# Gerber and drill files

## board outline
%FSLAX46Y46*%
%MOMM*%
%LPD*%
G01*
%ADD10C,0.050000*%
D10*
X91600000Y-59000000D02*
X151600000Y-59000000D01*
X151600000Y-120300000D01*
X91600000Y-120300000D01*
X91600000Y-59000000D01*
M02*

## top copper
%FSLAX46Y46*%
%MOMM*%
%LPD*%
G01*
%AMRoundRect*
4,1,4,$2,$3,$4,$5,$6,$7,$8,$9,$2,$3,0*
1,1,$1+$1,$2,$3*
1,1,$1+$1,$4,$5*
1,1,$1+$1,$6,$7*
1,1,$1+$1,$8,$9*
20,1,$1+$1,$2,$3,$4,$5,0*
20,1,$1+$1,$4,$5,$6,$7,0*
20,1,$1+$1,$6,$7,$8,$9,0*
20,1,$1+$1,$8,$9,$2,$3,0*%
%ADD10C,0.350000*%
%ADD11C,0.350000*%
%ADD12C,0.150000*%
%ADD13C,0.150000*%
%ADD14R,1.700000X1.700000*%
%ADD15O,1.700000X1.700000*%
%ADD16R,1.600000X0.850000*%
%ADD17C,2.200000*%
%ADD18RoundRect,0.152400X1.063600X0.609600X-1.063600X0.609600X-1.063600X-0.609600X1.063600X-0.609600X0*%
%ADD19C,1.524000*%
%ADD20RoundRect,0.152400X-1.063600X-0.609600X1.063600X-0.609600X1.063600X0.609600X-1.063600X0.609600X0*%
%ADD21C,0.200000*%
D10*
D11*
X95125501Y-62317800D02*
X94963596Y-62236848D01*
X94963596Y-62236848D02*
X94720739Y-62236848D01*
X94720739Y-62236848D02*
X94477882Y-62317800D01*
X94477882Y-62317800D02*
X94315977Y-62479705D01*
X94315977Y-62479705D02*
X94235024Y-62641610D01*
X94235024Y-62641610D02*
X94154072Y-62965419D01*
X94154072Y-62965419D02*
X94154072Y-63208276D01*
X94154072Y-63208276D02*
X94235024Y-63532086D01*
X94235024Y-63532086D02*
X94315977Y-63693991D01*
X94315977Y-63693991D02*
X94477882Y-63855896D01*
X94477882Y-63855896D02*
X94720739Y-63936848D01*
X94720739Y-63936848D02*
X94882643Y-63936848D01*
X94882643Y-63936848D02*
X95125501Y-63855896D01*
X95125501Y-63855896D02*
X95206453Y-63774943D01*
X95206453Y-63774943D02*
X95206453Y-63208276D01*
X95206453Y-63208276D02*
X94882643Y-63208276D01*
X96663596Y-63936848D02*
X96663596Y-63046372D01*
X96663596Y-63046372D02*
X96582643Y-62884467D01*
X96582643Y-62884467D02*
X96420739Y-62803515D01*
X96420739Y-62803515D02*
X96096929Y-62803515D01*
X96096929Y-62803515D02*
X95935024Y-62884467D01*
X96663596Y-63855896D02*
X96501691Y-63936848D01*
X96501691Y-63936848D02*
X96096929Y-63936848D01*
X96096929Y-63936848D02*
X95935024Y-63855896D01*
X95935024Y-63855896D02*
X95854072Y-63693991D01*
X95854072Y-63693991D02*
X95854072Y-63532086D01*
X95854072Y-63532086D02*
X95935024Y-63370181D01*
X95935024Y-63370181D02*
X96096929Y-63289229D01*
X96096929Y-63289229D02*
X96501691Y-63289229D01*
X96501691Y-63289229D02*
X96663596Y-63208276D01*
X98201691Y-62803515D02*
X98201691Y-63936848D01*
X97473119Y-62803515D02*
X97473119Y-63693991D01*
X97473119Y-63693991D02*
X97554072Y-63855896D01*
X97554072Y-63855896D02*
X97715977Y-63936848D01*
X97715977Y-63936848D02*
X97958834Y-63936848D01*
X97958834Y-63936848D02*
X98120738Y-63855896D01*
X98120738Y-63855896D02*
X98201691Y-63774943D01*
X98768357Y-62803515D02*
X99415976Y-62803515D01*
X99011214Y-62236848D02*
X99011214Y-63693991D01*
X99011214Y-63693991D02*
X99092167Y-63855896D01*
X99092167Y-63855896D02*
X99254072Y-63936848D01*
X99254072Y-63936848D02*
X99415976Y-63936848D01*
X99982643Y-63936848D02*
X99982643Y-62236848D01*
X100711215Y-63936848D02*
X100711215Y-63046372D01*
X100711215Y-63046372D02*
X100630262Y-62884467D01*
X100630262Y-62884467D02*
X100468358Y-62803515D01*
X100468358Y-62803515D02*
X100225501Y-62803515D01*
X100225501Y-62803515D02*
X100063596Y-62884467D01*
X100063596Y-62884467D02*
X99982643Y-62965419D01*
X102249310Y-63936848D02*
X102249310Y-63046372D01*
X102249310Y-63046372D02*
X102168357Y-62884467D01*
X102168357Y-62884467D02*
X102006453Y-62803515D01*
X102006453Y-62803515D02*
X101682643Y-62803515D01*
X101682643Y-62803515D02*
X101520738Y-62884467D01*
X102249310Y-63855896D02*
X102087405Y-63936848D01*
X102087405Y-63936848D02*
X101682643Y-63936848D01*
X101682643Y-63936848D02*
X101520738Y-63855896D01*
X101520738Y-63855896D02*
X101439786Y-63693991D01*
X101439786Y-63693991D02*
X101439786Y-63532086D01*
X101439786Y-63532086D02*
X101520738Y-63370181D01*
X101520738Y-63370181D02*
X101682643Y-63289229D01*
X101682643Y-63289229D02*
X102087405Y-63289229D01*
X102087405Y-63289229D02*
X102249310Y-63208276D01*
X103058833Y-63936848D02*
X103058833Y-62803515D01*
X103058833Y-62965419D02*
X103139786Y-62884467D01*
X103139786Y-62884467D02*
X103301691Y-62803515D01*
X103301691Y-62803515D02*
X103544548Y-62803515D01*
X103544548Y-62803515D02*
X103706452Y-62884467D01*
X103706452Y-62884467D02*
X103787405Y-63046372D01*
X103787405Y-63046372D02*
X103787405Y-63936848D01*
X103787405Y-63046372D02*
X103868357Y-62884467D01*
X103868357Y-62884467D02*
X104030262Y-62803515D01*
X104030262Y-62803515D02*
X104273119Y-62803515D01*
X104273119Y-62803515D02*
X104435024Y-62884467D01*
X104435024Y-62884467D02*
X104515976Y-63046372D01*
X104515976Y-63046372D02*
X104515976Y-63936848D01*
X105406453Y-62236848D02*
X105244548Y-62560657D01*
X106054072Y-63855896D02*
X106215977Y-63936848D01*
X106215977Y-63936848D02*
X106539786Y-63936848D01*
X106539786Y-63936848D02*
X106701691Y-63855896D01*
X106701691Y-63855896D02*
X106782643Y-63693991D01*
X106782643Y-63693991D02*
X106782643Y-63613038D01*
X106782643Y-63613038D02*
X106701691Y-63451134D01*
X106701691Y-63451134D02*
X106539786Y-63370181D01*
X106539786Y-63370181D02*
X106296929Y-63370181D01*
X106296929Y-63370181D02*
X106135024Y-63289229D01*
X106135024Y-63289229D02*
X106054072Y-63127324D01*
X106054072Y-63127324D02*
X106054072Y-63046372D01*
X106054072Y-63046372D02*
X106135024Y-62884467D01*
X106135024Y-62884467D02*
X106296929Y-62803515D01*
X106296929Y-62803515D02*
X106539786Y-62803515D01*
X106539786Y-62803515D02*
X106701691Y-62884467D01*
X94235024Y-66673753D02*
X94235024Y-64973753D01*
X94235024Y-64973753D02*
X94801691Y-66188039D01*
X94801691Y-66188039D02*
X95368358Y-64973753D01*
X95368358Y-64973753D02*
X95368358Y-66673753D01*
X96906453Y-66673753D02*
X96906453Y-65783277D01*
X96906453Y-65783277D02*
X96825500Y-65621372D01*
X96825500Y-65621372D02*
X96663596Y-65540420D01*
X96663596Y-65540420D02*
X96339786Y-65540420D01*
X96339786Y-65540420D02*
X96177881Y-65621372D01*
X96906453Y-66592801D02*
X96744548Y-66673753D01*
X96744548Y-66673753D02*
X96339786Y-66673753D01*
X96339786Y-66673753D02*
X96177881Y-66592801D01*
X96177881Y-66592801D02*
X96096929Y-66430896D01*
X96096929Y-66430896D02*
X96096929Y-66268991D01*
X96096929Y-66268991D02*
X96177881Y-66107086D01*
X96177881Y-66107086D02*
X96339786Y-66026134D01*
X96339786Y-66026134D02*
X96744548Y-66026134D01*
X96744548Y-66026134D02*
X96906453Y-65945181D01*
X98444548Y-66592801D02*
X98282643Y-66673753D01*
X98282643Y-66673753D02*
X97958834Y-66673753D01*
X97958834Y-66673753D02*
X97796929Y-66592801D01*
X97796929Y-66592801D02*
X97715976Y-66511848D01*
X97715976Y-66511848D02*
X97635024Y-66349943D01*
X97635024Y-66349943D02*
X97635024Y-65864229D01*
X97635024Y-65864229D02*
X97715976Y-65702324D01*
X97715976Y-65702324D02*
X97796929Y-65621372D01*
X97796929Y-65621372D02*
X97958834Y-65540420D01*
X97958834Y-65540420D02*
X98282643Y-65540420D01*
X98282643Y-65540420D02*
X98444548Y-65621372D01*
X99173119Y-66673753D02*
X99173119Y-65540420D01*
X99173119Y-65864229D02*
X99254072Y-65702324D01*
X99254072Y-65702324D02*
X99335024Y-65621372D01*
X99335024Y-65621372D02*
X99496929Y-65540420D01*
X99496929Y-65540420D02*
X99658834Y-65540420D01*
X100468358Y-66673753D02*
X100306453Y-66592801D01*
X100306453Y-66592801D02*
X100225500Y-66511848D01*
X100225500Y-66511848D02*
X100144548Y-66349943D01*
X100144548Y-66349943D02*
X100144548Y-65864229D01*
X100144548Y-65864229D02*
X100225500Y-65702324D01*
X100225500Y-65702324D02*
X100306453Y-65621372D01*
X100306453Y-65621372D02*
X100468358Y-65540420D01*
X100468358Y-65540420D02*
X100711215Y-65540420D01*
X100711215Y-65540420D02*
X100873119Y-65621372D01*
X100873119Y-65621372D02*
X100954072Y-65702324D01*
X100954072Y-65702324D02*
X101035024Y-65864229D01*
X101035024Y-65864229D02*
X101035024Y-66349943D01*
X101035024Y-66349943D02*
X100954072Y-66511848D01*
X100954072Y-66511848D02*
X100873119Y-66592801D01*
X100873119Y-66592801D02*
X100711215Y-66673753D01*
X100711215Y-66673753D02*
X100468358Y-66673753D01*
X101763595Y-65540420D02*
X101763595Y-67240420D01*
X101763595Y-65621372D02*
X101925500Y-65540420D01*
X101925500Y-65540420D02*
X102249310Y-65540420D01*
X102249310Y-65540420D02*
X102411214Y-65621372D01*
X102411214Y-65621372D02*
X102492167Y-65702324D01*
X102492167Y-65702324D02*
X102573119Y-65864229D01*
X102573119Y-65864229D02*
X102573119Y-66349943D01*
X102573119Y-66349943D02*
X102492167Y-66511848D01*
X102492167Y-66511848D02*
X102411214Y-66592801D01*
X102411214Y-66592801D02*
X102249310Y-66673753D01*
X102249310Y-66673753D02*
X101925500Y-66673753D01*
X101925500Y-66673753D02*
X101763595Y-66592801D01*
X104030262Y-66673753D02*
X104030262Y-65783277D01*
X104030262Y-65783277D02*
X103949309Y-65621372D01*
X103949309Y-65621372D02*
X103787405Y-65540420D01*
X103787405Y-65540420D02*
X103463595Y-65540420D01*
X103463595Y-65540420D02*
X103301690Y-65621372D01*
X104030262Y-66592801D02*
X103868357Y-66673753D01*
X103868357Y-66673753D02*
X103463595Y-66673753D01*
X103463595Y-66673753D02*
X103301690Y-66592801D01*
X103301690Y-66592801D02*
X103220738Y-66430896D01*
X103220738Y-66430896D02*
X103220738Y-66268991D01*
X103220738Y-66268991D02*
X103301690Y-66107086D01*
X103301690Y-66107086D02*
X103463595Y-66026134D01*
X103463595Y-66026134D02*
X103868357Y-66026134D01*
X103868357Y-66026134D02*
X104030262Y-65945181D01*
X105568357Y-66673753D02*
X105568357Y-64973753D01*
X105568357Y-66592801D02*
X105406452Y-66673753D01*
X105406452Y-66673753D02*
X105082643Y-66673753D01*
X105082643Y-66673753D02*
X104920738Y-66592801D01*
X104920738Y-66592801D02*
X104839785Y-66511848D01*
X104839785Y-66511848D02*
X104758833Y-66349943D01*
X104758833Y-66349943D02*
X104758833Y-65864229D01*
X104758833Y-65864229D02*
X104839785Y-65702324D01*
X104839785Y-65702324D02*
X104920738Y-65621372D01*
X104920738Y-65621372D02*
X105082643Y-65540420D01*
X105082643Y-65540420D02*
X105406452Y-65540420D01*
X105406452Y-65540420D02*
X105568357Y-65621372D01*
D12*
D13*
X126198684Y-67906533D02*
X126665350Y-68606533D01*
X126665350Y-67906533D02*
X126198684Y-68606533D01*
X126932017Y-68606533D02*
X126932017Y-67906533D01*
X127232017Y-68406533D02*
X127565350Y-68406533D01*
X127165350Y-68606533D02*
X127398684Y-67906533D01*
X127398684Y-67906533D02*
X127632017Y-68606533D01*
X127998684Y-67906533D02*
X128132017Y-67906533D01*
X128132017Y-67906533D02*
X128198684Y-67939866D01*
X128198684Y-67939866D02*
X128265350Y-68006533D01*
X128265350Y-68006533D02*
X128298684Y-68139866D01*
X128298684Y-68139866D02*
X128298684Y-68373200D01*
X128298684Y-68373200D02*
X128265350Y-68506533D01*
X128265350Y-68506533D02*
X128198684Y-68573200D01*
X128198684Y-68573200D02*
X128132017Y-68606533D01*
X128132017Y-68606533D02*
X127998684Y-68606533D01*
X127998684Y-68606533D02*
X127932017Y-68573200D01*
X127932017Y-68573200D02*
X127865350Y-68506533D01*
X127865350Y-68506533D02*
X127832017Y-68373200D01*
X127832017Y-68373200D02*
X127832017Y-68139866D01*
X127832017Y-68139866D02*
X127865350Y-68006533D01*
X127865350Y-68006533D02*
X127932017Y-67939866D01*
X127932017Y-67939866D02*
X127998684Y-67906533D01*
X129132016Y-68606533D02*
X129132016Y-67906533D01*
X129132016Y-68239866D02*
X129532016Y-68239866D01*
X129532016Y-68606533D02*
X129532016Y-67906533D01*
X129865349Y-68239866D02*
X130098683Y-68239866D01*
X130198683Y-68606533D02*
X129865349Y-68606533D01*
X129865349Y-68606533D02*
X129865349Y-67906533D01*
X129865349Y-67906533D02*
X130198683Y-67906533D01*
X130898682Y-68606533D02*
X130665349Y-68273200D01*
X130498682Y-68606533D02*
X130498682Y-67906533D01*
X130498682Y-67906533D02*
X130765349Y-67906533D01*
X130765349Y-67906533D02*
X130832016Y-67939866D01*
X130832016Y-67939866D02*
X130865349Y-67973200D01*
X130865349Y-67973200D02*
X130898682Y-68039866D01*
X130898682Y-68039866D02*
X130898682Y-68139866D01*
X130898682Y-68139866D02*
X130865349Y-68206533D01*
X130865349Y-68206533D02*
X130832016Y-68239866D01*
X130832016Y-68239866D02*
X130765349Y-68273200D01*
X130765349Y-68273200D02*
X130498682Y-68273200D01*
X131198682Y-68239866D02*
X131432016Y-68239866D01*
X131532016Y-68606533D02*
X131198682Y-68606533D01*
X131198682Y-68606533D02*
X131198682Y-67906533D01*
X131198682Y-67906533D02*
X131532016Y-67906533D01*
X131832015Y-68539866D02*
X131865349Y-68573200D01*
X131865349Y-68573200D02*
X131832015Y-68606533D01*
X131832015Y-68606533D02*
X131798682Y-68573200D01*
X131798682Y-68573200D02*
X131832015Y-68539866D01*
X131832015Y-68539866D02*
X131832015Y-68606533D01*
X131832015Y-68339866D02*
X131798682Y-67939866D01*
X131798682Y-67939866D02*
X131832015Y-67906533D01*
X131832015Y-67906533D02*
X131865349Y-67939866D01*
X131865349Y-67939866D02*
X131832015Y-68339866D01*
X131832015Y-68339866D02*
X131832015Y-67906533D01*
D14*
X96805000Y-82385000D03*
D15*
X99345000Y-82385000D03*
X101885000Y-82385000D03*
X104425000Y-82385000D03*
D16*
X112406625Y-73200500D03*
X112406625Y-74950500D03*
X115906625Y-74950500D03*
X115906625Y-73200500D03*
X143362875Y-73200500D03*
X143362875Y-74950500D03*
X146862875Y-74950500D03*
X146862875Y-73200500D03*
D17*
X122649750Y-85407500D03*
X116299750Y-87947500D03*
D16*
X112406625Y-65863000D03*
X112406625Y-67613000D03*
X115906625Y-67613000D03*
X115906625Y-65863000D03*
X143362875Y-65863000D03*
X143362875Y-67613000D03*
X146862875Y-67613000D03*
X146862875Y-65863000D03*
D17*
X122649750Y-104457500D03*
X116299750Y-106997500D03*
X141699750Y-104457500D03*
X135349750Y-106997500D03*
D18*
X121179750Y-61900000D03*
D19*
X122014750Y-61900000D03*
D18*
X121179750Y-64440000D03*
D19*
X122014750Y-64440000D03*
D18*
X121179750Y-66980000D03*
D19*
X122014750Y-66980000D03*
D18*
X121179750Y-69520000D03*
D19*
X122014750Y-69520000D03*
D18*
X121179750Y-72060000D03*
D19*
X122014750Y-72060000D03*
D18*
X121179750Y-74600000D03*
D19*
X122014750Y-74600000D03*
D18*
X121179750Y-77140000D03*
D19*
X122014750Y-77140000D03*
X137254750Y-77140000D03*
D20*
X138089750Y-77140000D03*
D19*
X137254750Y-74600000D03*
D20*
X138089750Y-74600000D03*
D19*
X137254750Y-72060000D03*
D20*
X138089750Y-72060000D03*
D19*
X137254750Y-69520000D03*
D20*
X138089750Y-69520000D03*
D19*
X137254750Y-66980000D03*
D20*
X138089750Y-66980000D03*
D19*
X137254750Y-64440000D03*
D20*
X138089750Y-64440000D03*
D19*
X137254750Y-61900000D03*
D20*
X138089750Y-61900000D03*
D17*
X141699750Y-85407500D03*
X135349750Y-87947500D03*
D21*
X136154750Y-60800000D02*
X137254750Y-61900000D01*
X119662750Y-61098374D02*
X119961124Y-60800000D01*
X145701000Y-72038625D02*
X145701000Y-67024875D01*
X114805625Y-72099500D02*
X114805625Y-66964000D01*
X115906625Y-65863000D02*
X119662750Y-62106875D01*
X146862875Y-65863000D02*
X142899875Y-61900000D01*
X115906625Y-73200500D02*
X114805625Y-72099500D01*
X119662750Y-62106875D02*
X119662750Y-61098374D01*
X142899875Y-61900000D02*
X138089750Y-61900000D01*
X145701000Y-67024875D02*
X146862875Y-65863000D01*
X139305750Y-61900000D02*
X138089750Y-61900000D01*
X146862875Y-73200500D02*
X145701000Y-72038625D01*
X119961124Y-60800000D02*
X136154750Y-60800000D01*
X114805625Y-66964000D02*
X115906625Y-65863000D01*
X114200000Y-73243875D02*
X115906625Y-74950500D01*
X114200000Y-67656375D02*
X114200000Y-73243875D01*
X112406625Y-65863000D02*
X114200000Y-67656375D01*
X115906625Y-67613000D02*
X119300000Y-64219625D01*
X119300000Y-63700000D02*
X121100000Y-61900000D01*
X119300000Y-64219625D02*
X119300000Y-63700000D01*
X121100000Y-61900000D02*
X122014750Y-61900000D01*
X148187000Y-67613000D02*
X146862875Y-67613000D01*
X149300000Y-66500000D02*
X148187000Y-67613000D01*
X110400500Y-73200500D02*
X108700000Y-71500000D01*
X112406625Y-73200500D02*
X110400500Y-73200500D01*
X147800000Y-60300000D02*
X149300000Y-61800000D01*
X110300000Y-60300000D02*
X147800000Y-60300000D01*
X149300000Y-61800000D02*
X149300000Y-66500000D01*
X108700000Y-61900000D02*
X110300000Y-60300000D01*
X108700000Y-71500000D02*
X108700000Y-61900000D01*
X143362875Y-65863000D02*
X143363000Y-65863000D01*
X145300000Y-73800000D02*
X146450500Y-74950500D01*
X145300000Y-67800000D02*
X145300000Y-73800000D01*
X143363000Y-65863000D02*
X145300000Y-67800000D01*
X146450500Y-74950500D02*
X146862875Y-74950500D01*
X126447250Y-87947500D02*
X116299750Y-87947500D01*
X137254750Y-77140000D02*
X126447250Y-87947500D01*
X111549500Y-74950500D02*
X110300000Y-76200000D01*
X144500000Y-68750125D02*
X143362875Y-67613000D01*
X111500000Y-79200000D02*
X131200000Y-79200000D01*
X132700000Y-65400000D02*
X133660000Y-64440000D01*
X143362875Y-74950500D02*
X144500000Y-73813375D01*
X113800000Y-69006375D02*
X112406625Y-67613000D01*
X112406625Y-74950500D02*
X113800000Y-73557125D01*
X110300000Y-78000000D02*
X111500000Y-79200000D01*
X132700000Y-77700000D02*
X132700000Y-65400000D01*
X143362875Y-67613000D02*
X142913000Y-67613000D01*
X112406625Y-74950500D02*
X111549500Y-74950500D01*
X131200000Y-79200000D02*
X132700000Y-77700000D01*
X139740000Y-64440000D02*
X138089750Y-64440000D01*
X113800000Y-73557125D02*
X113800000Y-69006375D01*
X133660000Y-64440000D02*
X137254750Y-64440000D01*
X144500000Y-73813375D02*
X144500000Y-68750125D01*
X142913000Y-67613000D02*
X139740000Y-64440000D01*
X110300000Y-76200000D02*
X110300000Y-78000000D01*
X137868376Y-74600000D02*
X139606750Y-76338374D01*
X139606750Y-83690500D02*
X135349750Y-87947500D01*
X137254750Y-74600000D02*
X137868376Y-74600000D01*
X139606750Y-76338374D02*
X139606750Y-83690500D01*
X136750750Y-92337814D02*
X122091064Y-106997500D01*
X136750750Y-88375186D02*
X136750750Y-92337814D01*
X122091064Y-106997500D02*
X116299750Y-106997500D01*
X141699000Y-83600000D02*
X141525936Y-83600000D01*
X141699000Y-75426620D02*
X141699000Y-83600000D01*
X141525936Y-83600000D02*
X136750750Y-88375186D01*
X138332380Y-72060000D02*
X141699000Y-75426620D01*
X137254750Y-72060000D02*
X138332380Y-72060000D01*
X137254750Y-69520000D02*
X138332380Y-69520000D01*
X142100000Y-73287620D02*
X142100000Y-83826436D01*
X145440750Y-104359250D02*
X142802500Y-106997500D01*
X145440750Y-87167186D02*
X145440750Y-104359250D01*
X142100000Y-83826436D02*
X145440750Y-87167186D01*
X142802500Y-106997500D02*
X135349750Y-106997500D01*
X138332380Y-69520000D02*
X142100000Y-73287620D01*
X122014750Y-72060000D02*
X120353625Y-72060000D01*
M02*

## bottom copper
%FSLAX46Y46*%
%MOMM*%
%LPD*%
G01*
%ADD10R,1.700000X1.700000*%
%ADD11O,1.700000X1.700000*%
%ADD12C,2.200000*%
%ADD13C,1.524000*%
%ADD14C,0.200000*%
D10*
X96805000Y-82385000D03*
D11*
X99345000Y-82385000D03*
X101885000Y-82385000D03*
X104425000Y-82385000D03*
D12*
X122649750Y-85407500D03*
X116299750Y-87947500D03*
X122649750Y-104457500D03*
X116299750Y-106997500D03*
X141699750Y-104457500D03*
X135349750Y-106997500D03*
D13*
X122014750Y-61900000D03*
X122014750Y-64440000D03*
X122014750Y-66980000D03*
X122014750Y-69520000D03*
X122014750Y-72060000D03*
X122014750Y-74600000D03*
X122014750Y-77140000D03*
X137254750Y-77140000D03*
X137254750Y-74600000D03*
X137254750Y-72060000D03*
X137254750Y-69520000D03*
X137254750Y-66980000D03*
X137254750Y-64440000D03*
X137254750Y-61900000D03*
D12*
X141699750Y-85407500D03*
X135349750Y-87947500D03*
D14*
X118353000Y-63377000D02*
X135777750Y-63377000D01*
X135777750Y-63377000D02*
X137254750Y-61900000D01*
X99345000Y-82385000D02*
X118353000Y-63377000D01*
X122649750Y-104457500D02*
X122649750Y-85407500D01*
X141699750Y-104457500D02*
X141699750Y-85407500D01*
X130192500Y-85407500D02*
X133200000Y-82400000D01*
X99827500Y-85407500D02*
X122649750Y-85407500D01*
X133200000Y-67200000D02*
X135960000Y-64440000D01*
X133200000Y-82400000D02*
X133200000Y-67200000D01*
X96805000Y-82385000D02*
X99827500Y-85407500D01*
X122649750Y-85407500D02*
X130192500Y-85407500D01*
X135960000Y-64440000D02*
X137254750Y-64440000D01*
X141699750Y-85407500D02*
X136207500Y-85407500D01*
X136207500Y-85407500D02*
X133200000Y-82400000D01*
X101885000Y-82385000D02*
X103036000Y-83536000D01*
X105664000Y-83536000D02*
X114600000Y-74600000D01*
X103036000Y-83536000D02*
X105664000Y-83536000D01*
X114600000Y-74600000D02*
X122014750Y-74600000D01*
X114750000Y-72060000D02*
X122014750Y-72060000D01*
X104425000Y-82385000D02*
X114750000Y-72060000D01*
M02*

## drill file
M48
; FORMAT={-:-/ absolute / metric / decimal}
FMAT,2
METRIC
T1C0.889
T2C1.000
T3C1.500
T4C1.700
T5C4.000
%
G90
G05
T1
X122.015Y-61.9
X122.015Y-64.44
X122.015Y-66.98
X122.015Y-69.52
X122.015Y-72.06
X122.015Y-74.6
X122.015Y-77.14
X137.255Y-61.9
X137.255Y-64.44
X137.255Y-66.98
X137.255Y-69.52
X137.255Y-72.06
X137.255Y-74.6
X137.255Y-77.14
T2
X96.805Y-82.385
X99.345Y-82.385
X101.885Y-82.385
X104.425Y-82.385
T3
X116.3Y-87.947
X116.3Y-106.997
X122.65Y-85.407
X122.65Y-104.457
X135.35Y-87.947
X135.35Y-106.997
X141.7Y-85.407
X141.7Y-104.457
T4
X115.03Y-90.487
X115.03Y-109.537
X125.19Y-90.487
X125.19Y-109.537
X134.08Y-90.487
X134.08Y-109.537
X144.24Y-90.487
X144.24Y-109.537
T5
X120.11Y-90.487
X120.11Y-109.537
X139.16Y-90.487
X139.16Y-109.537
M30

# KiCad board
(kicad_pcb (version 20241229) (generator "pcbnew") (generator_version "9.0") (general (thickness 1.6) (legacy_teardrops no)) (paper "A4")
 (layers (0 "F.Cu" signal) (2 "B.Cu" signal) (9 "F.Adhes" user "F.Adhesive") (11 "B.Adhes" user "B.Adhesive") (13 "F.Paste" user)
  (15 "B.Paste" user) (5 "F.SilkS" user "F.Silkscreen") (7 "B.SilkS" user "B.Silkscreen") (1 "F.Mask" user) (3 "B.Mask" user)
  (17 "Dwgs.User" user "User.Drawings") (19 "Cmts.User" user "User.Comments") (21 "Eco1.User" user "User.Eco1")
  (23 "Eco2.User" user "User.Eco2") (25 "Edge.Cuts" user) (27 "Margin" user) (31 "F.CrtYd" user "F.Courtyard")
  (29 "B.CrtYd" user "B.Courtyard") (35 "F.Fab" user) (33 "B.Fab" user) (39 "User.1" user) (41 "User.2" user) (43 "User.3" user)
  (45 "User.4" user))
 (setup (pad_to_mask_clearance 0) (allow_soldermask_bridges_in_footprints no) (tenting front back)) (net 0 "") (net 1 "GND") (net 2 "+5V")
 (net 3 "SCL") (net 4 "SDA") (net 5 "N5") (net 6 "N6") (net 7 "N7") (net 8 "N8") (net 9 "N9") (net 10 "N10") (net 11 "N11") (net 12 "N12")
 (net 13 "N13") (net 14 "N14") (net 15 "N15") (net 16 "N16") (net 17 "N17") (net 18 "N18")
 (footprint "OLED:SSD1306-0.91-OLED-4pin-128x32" (layer "F.Cu") (at 94.615 118.885 90)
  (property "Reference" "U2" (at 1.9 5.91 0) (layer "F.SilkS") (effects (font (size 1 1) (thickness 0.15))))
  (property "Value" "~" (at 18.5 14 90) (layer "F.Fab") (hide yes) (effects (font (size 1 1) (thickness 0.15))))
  (pad "1" thru_hole rect (at 36.5 2.19 90) (size 1.7 1.7) (drill 1) (layers "*.Cu" "*.Mask") (remove_unused_layers no) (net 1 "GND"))
  (pad "2" thru_hole oval (at 36.5 4.73 90) (size 1.7 1.7) (drill 1) (layers "*.Cu" "*.Mask") (remove_unused_layers no) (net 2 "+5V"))
  (pad "3" thru_hole oval (at 36.5 7.27 90) (size 1.7 1.7) (drill 1) (layers "*.Cu" "*.Mask") (remove_unused_layers no) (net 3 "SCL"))
  (pad "4" thru_hole oval (at 36.5 9.81 90) (size 1.7 1.7) (drill 1) (layers "*.Cu" "*.Mask") (remove_unused_layers no) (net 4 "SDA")))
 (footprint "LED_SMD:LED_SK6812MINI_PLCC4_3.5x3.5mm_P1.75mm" (layer "F.Cu") (at 114.156625 74.0755)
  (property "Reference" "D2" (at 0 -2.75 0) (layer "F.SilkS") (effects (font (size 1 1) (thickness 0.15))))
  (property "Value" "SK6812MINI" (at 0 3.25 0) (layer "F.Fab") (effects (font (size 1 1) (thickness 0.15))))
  (pad "1" smd rect (at -1.75 -0.875) (size 1.6 0.85) (layers "F.Cu" "F.Mask" "F.Paste") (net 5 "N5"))
  (pad "2" smd rect (at -1.75 0.875) (size 1.6 0.85) (layers "F.Cu" "F.Mask" "F.Paste") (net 1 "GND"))
  (pad "3" smd rect (at 1.75 0.875) (size 1.6 0.85) (layers "F.Cu" "F.Mask" "F.Paste") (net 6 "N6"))
  (pad "4" smd rect (at 1.75 -0.875) (size 1.6 0.85) (layers "F.Cu" "F.Mask" "F.Paste") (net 2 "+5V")))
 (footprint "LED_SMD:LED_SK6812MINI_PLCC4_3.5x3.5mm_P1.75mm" (layer "F.Cu") (at 145.112875 74.0755)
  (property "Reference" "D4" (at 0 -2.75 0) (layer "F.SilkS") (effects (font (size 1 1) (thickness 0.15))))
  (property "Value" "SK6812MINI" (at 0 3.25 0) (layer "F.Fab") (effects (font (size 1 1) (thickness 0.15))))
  (pad "1" smd rect (at -1.75 -0.875) (size 1.6 0.85) (layers "F.Cu" "F.Mask" "F.Paste") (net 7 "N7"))
  (pad "2" smd rect (at -1.75 0.875) (size 1.6 0.85) (layers "F.Cu" "F.Mask" "F.Paste") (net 1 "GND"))
  (pad "3" smd rect (at 1.75 0.875) (size 1.6 0.85) (layers "F.Cu" "F.Mask" "F.Paste") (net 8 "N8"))
  (pad "4" smd rect (at 1.75 -0.875) (size 1.6 0.85) (layers "F.Cu" "F.Mask" "F.Paste") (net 2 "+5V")))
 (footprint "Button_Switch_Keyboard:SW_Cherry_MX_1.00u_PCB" (layer "F.Cu") (at 122.64975 85.4075)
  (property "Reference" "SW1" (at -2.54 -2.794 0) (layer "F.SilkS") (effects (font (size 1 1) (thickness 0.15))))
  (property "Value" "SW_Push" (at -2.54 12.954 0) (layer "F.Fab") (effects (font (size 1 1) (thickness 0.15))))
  (pad "" np_thru_hole circle (at -7.62 5.08) (size 1.7 1.7) (drill 1.7) (layers "*.Cu" "*.Mask"))
  (pad "" np_thru_hole circle (at -2.54 5.08) (size 4 4) (drill 4) (layers "*.Cu" "*.Mask"))
  (pad "" np_thru_hole circle (at 2.54 5.08) (size 1.7 1.7) (drill 1.7) (layers "*.Cu" "*.Mask"))
  (pad "1" thru_hole circle (at 0 0) (size 2.2 2.2) (drill 1.5) (layers "*.Cu" "*.Mask") (remove_unused_layers no) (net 1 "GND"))
  (pad "2" thru_hole circle (at -6.35 2.54) (size 2.2 2.2) (drill 1.5) (layers "*.Cu" "*.Mask") (remove_unused_layers no) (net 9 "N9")))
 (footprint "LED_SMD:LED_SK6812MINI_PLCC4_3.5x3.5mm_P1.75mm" (layer "F.Cu") (at 114.156625 66.738)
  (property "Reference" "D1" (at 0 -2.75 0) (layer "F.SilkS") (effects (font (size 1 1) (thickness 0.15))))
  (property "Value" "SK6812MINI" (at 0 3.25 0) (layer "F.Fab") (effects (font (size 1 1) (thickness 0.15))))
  (pad "1" smd rect (at -1.75 -0.875) (size 1.6 0.85) (layers "F.Cu" "F.Mask" "F.Paste") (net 6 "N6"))
  (pad "2" smd rect (at -1.75 0.875) (size 1.6 0.85) (layers "F.Cu" "F.Mask" "F.Paste") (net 1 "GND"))
  (pad "3" smd rect (at 1.75 0.875) (size 1.6 0.85) (layers "F.Cu" "F.Mask" "F.Paste") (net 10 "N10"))
  (pad "4" smd rect (at 1.75 -0.875) (size 1.6 0.85) (layers "F.Cu" "F.Mask" "F.Paste") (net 2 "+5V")))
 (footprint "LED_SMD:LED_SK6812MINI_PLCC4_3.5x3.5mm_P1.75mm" (layer "F.Cu") (at 145.112875 66.738)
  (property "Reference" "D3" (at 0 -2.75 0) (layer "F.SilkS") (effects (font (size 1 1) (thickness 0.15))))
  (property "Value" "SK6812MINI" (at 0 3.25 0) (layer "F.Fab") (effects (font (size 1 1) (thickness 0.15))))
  (pad "1" smd rect (at -1.75 -0.875) (size 1.6 0.85) (layers "F.Cu" "F.Mask" "F.Paste") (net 8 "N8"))
  (pad "2" smd rect (at -1.75 0.875) (size 1.6 0.85) (layers "F.Cu" "F.Mask" "F.Paste") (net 1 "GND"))
  (pad "3" smd rect (at 1.75 0.875) (size 1.6 0.85) (layers "F.Cu" "F.Mask" "F.Paste") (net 5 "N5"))
  (pad "4" smd rect (at 1.75 -0.875) (size 1.6 0.85) (layers "F.Cu" "F.Mask" "F.Paste") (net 2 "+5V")))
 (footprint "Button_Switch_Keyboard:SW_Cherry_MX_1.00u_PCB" (layer "F.Cu") (at 122.64975 104.4575)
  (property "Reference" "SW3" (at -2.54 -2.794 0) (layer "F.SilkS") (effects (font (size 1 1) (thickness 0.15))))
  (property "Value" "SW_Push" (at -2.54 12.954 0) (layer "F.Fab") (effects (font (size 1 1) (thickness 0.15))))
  (pad "" np_thru_hole circle (at -7.62 5.08) (size 1.7 1.7) (drill 1.7) (layers "*.Cu" "*.Mask"))
  (pad "" np_thru_hole circle (at -2.54 5.08) (size 4 4) (drill 4) (layers "*.Cu" "*.Mask"))
  (pad "" np_thru_hole circle (at 2.54 5.08) (size 1.7 1.7) (drill 1.7) (layers "*.Cu" "*.Mask"))
  (pad "1" thru_hole circle (at 0 0) (size 2.2 2.2) (drill 1.5) (layers "*.Cu" "*.Mask") (remove_unused_layers no) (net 1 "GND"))
  (pad "2" thru_hole circle (at -6.35 2.54) (size 2.2 2.2) (drill 1.5) (layers "*.Cu" "*.Mask") (remove_unused_layers no) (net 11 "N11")))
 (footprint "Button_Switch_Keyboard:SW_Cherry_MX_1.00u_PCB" (layer "F.Cu") (at 141.69975 104.4575)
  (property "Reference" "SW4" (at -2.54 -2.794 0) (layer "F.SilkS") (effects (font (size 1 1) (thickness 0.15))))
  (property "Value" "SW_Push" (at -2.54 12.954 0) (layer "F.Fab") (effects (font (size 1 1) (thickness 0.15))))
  (pad "" np_thru_hole circle (at -7.62 5.08) (size 1.7 1.7) (drill 1.7) (layers "*.Cu" "*.Mask"))
  (pad "" np_thru_hole circle (at -2.54 5.08) (size 4 4) (drill 4) (layers "*.Cu" "*.Mask"))
  (pad "" np_thru_hole circle (at 2.54 5.08) (size 1.7 1.7) (drill 1.7) (layers "*.Cu" "*.Mask"))
  (pad "1" thru_hole circle (at 0 0) (size 2.2 2.2) (drill 1.5) (layers "*.Cu" "*.Mask") (remove_unused_layers no) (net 1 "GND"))
  (pad "2" thru_hole circle (at -6.35 2.54) (size 2.2 2.2) (drill 1.5) (layers "*.Cu" "*.Mask") (remove_unused_layers no) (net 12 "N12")))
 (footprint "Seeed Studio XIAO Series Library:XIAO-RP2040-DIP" (layer "F.Cu") (at 129.63475 69.52)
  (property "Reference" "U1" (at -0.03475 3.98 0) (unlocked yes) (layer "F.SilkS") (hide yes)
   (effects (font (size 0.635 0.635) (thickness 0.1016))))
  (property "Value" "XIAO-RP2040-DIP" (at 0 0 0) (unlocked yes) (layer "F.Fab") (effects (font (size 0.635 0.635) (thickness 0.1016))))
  (pad "1" smd roundrect (at -8.455 -7.62 180) (size 2.432 1.524) (layers "F.Cu" "F.Mask") (roundrect_rratio 0.1) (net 10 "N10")
   (thermal_bridge_angle 45))
  (pad "1" thru_hole circle (at -7.62 -7.62 180) (size 1.524 1.524) (drill 0.889) (layers "*.Cu" "*.Mask") (remove_unused_layers no)
   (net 10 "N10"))
  (pad "2" smd roundrect (at -8.455 -5.08 180) (size 2.432 1.524) (layers "F.Cu" "F.Mask") (roundrect_rratio 0.1) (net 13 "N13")
   (thermal_bridge_angle 45))
  (pad "2" thru_hole circle (at -7.62 -5.08 180) (size 1.524 1.524) (drill 0.889) (layers "*.Cu" "*.Mask") (remove_unused_layers no)
   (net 13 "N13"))
  (pad "3" smd roundrect (at -8.455 -2.54 180) (size 2.432 1.524) (layers "F.Cu" "F.Mask") (roundrect_rratio 0.1) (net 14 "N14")
   (thermal_bridge_angle 45))
  (pad "3" thru_hole circle (at -7.62 -2.54 180) (size 1.524 1.524) (drill 0.889) (layers "*.Cu" "*.Mask") (remove_unused_layers no)
   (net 14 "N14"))
  (pad "4" smd roundrect (at -8.455 0 180) (size 2.432 1.524) (layers "F.Cu" "F.Mask") (roundrect_rratio 0.1) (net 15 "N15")
   (thermal_bridge_angle 45))
  (pad "4" thru_hole circle (at -7.62 0 180) (size 1.524 1.524) (drill 0.889) (layers "*.Cu" "*.Mask") (remove_unused_layers no)
   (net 15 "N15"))
  (pad "5" smd roundrect (at -8.455 2.54 180) (size 2.432 1.524) (layers "F.Cu" "F.Mask") (roundrect_rratio 0.1) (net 4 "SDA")
   (thermal_bridge_angle 45))
  (pad "5" thru_hole circle (at -7.62 2.54 180) (size 1.524 1.524) (drill 0.889) (layers "*.Cu" "*.Mask") (remove_unused_layers no)
   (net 4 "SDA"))
  (pad "6" smd roundrect (at -8.455 5.08 180) (size 2.432 1.524) (layers "F.Cu" "F.Mask") (roundrect_rratio 0.1) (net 3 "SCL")
   (thermal_bridge_angle 45))
  (pad "6" thru_hole circle (at -7.62 5.08 180) (size 1.524 1.524) (drill 0.889) (layers "*.Cu" "*.Mask") (remove_unused_layers no)
   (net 3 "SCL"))
  (pad "7" smd roundrect (at -8.455 7.62 180) (size 2.432 1.524) (layers "F.Cu" "F.Mask") (roundrect_rratio 0.1) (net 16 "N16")
   (thermal_bridge_angle 45))
  (pad "7" thru_hole circle (at -7.62 7.62 180) (size 1.524 1.524) (drill 0.889) (layers "*.Cu" "*.Mask") (remove_unused_layers no)
   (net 16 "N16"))
  (pad "8" thru_hole circle (at 7.62 7.62) (size 1.524 1.524) (drill 0.889) (layers "*.Cu" "*.Mask") (remove_unused_layers no) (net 9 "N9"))
  (pad "8" smd roundrect (at 8.455 7.62) (size 2.432 1.524) (layers "F.Cu" "F.Mask") (roundrect_rratio 0.1) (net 9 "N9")
   (thermal_bridge_angle 45))
  (pad "9" thru_hole circle (at 7.62 5.08) (size 1.524 1.524) (drill 0.889) (layers "*.Cu" "*.Mask") (remove_unused_layers no)
   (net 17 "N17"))
  (pad "9" smd roundrect (at 8.455 5.08) (size 2.432 1.524) (layers "F.Cu" "F.Mask") (roundrect_rratio 0.1) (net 17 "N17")
   (thermal_bridge_angle 45))
  (pad "10" thru_hole circle (at 7.62 2.54) (size 1.524 1.524) (drill 0.889) (layers "*.Cu" "*.Mask") (remove_unused_layers no)
   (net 11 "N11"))
  (pad "10" smd roundrect (at 8.455 2.54) (size 2.432 1.524) (layers "F.Cu" "F.Mask") (roundrect_rratio 0.1) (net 11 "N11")
   (thermal_bridge_angle 45))
  (pad "11" thru_hole circle (at 7.62 0) (size 1.524 1.524) (drill 0.889) (layers "*.Cu" "*.Mask") (remove_unused_layers no) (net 12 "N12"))
  (pad "11" smd roundrect (at 8.455 0) (size 2.432 1.524) (layers "F.Cu" "F.Mask") (roundrect_rratio 0.1) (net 12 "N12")
   (thermal_bridge_angle 45))
  (pad "12" thru_hole circle (at 7.62 -2.54) (size 1.524 1.524) (drill 0.889) (layers "*.Cu" "*.Mask") (remove_unused_layers no)
   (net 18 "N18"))
  (pad "12" smd roundrect (at 8.455 -2.54) (size 2.432 1.524) (layers "F.Cu" "F.Mask") (roundrect_rratio 0.1) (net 18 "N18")
   (thermal_bridge_angle 45))
  (pad "13" thru_hole circle (at 7.62 -5.08) (size 1.524 1.524) (drill 0.889) (layers "*.Cu" "*.Mask") (remove_unused_layers no)
   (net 1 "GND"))
  (pad "13" smd roundrect (at 8.455 -5.08) (size 2.432 1.524) (layers "F.Cu" "F.Mask") (roundrect_rratio 0.1) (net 1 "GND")
   (thermal_bridge_angle 45))
  (pad "14" thru_hole circle (at 7.62 -7.62) (size 1.524 1.524) (drill 0.889) (layers "*.Cu" "*.Mask") (remove_unused_layers no)
   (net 2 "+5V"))
  (pad "14" smd roundrect (at 8.455 -7.62) (size 2.432 1.524) (layers "F.Cu" "F.Mask") (roundrect_rratio 0.1) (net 2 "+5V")
   (thermal_bridge_angle 45)))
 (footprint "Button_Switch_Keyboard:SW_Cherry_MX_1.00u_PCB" (layer "F.Cu") (at 141.69975 85.4075)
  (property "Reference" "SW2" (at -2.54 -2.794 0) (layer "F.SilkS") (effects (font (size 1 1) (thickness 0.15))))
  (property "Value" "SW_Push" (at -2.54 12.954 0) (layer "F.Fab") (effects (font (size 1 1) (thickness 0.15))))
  (pad "" np_thru_hole circle (at -7.62 5.08) (size 1.7 1.7) (drill 1.7) (layers "*.Cu" "*.Mask"))
  (pad "" np_thru_hole circle (at -2.54 5.08) (size 4 4) (drill 4) (layers "*.Cu" "*.Mask"))
  (pad "" np_thru_hole circle (at 2.54 5.08) (size 1.7 1.7) (drill 1.7) (layers "*.Cu" "*.Mask"))
  (pad "1" thru_hole circle (at 0 0) (size 2.2 2.2) (drill 1.5) (layers "*.Cu" "*.Mask") (remove_unused_layers no) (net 1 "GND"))
  (pad "2" thru_hole circle (at -6.35 2.54) (size 2.2 2.2) (drill 1.5) (layers "*.Cu" "*.Mask") (remove_unused_layers no) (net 17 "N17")))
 (gr_rect (start 91.6 59) (end 151.6 120.3) (stroke (width 0.05) (type default)) (fill no) (layer "Edge.Cuts"))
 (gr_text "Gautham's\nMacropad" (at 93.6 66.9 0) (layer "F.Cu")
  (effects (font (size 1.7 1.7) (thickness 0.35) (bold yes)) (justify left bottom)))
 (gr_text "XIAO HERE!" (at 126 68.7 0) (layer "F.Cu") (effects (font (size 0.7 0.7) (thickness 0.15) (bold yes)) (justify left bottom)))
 (segment (start 136.15475 60.8) (end 137.25475 61.9) (width 0.2) (layer "F.Cu") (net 2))
 (segment (start 119.66275 61.098374) (end 119.961124 60.8) (width 0.2) (layer "F.Cu") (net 2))
 (segment (start 145.701 72.038625) (end 145.701 67.024875) (width 0.2) (layer "F.Cu") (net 2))
 (segment (start 114.805625 72.0995) (end 114.805625 66.964) (width 0.2) (layer "F.Cu") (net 2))
 (segment (start 115.906625 65.863) (end 119.66275 62.106875) (width 0.2) (layer "F.Cu") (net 2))
 (segment (start 146.862875 65.863) (end 142.899875 61.9) (width 0.2) (layer "F.Cu") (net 2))
 (segment (start 115.906625 73.2005) (end 114.805625 72.0995) (width 0.2) (layer "F.Cu") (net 2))
 (segment (start 119.66275 62.106875) (end 119.66275 61.098374) (width 0.2) (layer "F.Cu") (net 2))
 (segment (start 142.899875 61.9) (end 138.08975 61.9) (width 0.2) (layer "F.Cu") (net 2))
 (segment (start 145.701 67.024875) (end 146.862875 65.863) (width 0.2) (layer "F.Cu") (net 2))
 (segment (start 139.30575 61.9) (end 138.08975 61.9) (width 0.2) (layer "F.Cu") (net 2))
 (segment (start 146.862875 73.2005) (end 145.701 72.038625) (width 0.2) (layer "F.Cu") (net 2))
 (segment (start 119.961124 60.8) (end 136.15475 60.8) (width 0.2) (layer "F.Cu") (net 2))
 (segment (start 114.805625 66.964) (end 115.906625 65.863) (width 0.2) (layer "F.Cu") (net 2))
 (segment (start 118.353 63.377) (end 135.77775 63.377) (width 0.2) (layer "B.Cu") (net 2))
 (segment (start 135.77775 63.377) (end 137.25475 61.9) (width 0.2) (layer "B.Cu") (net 2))
 (segment (start 99.345 82.385) (end 118.353 63.377) (width 0.2) (layer "B.Cu") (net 2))
 (segment (start 114.2 73.243875) (end 115.906625 74.9505) (width 0.2) (layer "F.Cu") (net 6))
 (segment (start 114.2 67.656375) (end 114.2 73.243875) (width 0.2) (layer "F.Cu") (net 6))
 (segment (start 112.406625 65.863) (end 114.2 67.656375) (width 0.2) (layer "F.Cu") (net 6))
 (segment (start 115.906625 67.613) (end 119.3 64.219625) (width 0.2) (layer "F.Cu") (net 10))
 (segment (start 119.3 63.7) (end 121.1 61.9) (width 0.2) (layer "F.Cu") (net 10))
 (segment (start 119.3 64.219625) (end 119.3 63.7) (width 0.2) (layer "F.Cu") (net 10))
 (segment (start 121.1 61.9) (end 122.01475 61.9) (width 0.2) (layer "F.Cu") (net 10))
 (segment (start 148.187 67.613) (end 146.862875 67.613) (width 0.2) (layer "F.Cu") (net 5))
 (segment (start 149.3 66.5) (end 148.187 67.613) (width 0.2) (layer "F.Cu") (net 5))
 (segment (start 110.4005 73.2005) (end 108.7 71.5) (width 0.2) (layer "F.Cu") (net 5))
 (segment (start 112.406625 73.2005) (end 110.4005 73.2005) (width 0.2) (layer "F.Cu") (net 5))
 (segment (start 147.8 60.3) (end 149.3 61.8) (width 0.2) (layer "F.Cu") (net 5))
 (segment (start 110.3 60.3) (end 147.8 60.3) (width 0.2) (layer "F.Cu") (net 5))
 (segment (start 149.3 61.8) (end 149.3 66.5) (width 0.2) (layer "F.Cu") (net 5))
 (segment (start 108.7 61.9) (end 110.3 60.3) (width 0.2) (layer "F.Cu") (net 5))
 (segment (start 108.7 71.5) (end 108.7 61.9) (width 0.2) (layer "F.Cu") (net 5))
 (segment (start 143.362875 65.863) (end 143.363 65.863) (width 0.2) (layer "F.Cu") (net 8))
 (segment (start 145.3 73.8) (end 146.4505 74.9505) (width 0.2) (layer "F.Cu") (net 8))
 (segment (start 145.3 67.8) (end 145.3 73.8) (width 0.2) (layer "F.Cu") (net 8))
 (segment (start 143.363 65.863) (end 145.3 67.8) (width 0.2) (layer "F.Cu") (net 8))
 (segment (start 146.4505 74.9505) (end 146.862875 74.9505) (width 0.2) (layer "F.Cu") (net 8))
 (segment (start 126.44725 87.9475) (end 116.29975 87.9475) (width 0.2) (layer "F.Cu") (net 9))
 (segment (start 137.25475 77.14) (end 126.44725 87.9475) (width 0.2) (layer "F.Cu") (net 9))
 (segment (start 111.5495 74.9505) (end 110.3 76.2) (width 0.2) (layer "F.Cu") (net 1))
 (segment (start 144.5 68.750125) (end 143.362875 67.613) (width 0.2) (layer "F.Cu") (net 1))
 (segment (start 111.5 79.2) (end 131.2 79.2) (width 0.2) (layer "F.Cu") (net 1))
 (segment (start 132.7 65.4) (end 133.66 64.44) (width 0.2) (layer "F.Cu") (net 1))
 (segment (start 143.362875 74.9505) (end 144.5 73.813375) (width 0.2) (layer "F.Cu") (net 1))
 (segment (start 113.8 69.006375) (end 112.406625 67.613) (width 0.2) (layer "F.Cu") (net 1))
 (segment (start 112.406625 74.9505) (end 113.8 73.557125) (width 0.2) (layer "F.Cu") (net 1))
 (segment (start 110.3 78) (end 111.5 79.2) (width 0.2) (layer "F.Cu") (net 1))
 (segment (start 132.7 77.7) (end 132.7 65.4) (width 0.2) (layer "F.Cu") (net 1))
 (segment (start 143.362875 67.613) (end 142.913 67.613) (width 0.2) (layer "F.Cu") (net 1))
 (segment (start 112.406625 74.9505) (end 111.5495 74.9505) (width 0.2) (layer "F.Cu") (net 1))
 (segment (start 131.2 79.2) (end 132.7 77.7) (width 0.2) (layer "F.Cu") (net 1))
 (segment (start 139.74 64.44) (end 138.08975 64.44) (width 0.2) (layer "F.Cu") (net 1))
 (segment (start 113.8 73.557125) (end 113.8 69.006375) (width 0.2) (layer "F.Cu") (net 1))
 (segment (start 133.66 64.44) (end 137.25475 64.44) (width 0.2) (layer "F.Cu") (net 1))
 (segment (start 144.5 73.813375) (end 144.5 68.750125) (width 0.2) (layer "F.Cu") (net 1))
 (segment (start 142.913 67.613) (end 139.74 64.44) (width 0.2) (layer "F.Cu") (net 1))
 (segment (start 110.3 76.2) (end 110.3 78) (width 0.2) (layer "F.Cu") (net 1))
 (segment (start 122.64975 104.4575) (end 122.64975 85.4075) (width 0.2) (layer "B.Cu") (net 1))
 (segment (start 141.69975 104.4575) (end 141.69975 85.4075) (width 0.2) (layer "B.Cu") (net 1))
 (segment (start 130.1925 85.4075) (end 133.2 82.4) (width 0.2) (layer "B.Cu") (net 1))
 (segment (start 99.8275 85.4075) (end 122.64975 85.4075) (width 0.2) (layer "B.Cu") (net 1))
 (segment (start 133.2 67.2) (end 135.96 64.44) (width 0.2) (layer "B.Cu") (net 1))
 (segment (start 133.2 82.4) (end 133.2 67.2) (width 0.2) (layer "B.Cu") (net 1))
 (segment (start 96.805 82.385) (end 99.8275 85.4075) (width 0.2) (layer "B.Cu") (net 1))
 (segment (start 122.64975 85.4075) (end 130.1925 85.4075) (width 0.2) (layer "B.Cu") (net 1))
 (segment (start 135.96 64.44) (end 137.25475 64.44) (width 0.2) (layer "B.Cu") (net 1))
 (segment (start 141.69975 85.4075) (end 136.2075 85.4075) (width 0.2) (layer "B.Cu") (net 1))
 (segment (start 136.2075 85.4075) (end 133.2 82.4) (width 0.2) (layer "B.Cu") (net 1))
 (segment (start 137.868376 74.6) (end 139.60675 76.338374) (width 0.2) (layer "F.Cu") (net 17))
 (segment (start 139.60675 83.6905) (end 135.34975 87.9475) (width 0.2) (layer "F.Cu") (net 17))
 (segment (start 137.25475 74.6) (end 137.868376 74.6) (width 0.2) (layer "F.Cu") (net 17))
 (segment (start 139.60675 76.338374) (end 139.60675 83.6905) (width 0.2) (layer "F.Cu") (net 17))
 (segment (start 136.75075 92.337814) (end 122.091064 106.9975) (width 0.2) (layer "F.Cu") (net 11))
 (segment (start 136.75075 88.375186) (end 136.75075 92.337814) (width 0.2) (layer "F.Cu") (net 11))
 (segment (start 122.091064 106.9975) (end 116.29975 106.9975) (width 0.2) (layer "F.Cu") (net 11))
 (segment (start 141.699 83.6) (end 141.525936 83.6) (width 0.2) (layer "F.Cu") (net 11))
 (segment (start 141.699 75.42662) (end 141.699 83.6) (width 0.2) (layer "F.Cu") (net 11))
 (segment (start 141.525936 83.6) (end 136.75075 88.375186) (width 0.2) (layer "F.Cu") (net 11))
 (segment (start 138.33238 72.06) (end 141.699 75.42662) (width 0.2) (layer "F.Cu") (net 11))
 (segment (start 137.25475 72.06) (end 138.33238 72.06) (width 0.2) (layer "F.Cu") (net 11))
 (segment (start 137.25475 69.52) (end 138.33238 69.52) (width 0.2) (layer "F.Cu") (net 12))
 (segment (start 142.1 73.28762) (end 142.1 83.826436) (width 0.2) (layer "F.Cu") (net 12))
 (segment (start 145.44075 104.35925) (end 142.8025 106.9975) (width 0.2) (layer "F.Cu") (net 12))
 (segment (start 145.44075 87.167186) (end 145.44075 104.35925) (width 0.2) (layer "F.Cu") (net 12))
 (segment (start 142.1 83.826436) (end 145.44075 87.167186) (width 0.2) (layer "F.Cu") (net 12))
 (segment (start 142.8025 106.9975) (end 135.34975 106.9975) (width 0.2) (layer "F.Cu") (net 12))
 (segment (start 138.33238 69.52) (end 142.1 73.28762) (width 0.2) (layer "F.Cu") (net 12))
 (segment (start 101.885 82.385) (end 103.036 83.536) (width 0.2) (layer "B.Cu") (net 3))
 (segment (start 105.664 83.536) (end 114.6 74.6) (width 0.2) (layer "B.Cu") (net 3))
 (segment (start 103.036 83.536) (end 105.664 83.536) (width 0.2) (layer "B.Cu") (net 3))
 (segment (start 114.6 74.6) (end 122.01475 74.6) (width 0.2) (layer "B.Cu") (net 3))
 (segment (start 122.01475 72.06) (end 120.353625 72.06) (width 0.2) (layer "F.Cu") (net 4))
 (segment (start 114.75 72.06) (end 122.01475 72.06) (width 0.2) (layer "B.Cu") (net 4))
 (segment (start 104.425 82.385) (end 114.75 72.06) (width 0.2) (layer "B.Cu") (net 4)))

